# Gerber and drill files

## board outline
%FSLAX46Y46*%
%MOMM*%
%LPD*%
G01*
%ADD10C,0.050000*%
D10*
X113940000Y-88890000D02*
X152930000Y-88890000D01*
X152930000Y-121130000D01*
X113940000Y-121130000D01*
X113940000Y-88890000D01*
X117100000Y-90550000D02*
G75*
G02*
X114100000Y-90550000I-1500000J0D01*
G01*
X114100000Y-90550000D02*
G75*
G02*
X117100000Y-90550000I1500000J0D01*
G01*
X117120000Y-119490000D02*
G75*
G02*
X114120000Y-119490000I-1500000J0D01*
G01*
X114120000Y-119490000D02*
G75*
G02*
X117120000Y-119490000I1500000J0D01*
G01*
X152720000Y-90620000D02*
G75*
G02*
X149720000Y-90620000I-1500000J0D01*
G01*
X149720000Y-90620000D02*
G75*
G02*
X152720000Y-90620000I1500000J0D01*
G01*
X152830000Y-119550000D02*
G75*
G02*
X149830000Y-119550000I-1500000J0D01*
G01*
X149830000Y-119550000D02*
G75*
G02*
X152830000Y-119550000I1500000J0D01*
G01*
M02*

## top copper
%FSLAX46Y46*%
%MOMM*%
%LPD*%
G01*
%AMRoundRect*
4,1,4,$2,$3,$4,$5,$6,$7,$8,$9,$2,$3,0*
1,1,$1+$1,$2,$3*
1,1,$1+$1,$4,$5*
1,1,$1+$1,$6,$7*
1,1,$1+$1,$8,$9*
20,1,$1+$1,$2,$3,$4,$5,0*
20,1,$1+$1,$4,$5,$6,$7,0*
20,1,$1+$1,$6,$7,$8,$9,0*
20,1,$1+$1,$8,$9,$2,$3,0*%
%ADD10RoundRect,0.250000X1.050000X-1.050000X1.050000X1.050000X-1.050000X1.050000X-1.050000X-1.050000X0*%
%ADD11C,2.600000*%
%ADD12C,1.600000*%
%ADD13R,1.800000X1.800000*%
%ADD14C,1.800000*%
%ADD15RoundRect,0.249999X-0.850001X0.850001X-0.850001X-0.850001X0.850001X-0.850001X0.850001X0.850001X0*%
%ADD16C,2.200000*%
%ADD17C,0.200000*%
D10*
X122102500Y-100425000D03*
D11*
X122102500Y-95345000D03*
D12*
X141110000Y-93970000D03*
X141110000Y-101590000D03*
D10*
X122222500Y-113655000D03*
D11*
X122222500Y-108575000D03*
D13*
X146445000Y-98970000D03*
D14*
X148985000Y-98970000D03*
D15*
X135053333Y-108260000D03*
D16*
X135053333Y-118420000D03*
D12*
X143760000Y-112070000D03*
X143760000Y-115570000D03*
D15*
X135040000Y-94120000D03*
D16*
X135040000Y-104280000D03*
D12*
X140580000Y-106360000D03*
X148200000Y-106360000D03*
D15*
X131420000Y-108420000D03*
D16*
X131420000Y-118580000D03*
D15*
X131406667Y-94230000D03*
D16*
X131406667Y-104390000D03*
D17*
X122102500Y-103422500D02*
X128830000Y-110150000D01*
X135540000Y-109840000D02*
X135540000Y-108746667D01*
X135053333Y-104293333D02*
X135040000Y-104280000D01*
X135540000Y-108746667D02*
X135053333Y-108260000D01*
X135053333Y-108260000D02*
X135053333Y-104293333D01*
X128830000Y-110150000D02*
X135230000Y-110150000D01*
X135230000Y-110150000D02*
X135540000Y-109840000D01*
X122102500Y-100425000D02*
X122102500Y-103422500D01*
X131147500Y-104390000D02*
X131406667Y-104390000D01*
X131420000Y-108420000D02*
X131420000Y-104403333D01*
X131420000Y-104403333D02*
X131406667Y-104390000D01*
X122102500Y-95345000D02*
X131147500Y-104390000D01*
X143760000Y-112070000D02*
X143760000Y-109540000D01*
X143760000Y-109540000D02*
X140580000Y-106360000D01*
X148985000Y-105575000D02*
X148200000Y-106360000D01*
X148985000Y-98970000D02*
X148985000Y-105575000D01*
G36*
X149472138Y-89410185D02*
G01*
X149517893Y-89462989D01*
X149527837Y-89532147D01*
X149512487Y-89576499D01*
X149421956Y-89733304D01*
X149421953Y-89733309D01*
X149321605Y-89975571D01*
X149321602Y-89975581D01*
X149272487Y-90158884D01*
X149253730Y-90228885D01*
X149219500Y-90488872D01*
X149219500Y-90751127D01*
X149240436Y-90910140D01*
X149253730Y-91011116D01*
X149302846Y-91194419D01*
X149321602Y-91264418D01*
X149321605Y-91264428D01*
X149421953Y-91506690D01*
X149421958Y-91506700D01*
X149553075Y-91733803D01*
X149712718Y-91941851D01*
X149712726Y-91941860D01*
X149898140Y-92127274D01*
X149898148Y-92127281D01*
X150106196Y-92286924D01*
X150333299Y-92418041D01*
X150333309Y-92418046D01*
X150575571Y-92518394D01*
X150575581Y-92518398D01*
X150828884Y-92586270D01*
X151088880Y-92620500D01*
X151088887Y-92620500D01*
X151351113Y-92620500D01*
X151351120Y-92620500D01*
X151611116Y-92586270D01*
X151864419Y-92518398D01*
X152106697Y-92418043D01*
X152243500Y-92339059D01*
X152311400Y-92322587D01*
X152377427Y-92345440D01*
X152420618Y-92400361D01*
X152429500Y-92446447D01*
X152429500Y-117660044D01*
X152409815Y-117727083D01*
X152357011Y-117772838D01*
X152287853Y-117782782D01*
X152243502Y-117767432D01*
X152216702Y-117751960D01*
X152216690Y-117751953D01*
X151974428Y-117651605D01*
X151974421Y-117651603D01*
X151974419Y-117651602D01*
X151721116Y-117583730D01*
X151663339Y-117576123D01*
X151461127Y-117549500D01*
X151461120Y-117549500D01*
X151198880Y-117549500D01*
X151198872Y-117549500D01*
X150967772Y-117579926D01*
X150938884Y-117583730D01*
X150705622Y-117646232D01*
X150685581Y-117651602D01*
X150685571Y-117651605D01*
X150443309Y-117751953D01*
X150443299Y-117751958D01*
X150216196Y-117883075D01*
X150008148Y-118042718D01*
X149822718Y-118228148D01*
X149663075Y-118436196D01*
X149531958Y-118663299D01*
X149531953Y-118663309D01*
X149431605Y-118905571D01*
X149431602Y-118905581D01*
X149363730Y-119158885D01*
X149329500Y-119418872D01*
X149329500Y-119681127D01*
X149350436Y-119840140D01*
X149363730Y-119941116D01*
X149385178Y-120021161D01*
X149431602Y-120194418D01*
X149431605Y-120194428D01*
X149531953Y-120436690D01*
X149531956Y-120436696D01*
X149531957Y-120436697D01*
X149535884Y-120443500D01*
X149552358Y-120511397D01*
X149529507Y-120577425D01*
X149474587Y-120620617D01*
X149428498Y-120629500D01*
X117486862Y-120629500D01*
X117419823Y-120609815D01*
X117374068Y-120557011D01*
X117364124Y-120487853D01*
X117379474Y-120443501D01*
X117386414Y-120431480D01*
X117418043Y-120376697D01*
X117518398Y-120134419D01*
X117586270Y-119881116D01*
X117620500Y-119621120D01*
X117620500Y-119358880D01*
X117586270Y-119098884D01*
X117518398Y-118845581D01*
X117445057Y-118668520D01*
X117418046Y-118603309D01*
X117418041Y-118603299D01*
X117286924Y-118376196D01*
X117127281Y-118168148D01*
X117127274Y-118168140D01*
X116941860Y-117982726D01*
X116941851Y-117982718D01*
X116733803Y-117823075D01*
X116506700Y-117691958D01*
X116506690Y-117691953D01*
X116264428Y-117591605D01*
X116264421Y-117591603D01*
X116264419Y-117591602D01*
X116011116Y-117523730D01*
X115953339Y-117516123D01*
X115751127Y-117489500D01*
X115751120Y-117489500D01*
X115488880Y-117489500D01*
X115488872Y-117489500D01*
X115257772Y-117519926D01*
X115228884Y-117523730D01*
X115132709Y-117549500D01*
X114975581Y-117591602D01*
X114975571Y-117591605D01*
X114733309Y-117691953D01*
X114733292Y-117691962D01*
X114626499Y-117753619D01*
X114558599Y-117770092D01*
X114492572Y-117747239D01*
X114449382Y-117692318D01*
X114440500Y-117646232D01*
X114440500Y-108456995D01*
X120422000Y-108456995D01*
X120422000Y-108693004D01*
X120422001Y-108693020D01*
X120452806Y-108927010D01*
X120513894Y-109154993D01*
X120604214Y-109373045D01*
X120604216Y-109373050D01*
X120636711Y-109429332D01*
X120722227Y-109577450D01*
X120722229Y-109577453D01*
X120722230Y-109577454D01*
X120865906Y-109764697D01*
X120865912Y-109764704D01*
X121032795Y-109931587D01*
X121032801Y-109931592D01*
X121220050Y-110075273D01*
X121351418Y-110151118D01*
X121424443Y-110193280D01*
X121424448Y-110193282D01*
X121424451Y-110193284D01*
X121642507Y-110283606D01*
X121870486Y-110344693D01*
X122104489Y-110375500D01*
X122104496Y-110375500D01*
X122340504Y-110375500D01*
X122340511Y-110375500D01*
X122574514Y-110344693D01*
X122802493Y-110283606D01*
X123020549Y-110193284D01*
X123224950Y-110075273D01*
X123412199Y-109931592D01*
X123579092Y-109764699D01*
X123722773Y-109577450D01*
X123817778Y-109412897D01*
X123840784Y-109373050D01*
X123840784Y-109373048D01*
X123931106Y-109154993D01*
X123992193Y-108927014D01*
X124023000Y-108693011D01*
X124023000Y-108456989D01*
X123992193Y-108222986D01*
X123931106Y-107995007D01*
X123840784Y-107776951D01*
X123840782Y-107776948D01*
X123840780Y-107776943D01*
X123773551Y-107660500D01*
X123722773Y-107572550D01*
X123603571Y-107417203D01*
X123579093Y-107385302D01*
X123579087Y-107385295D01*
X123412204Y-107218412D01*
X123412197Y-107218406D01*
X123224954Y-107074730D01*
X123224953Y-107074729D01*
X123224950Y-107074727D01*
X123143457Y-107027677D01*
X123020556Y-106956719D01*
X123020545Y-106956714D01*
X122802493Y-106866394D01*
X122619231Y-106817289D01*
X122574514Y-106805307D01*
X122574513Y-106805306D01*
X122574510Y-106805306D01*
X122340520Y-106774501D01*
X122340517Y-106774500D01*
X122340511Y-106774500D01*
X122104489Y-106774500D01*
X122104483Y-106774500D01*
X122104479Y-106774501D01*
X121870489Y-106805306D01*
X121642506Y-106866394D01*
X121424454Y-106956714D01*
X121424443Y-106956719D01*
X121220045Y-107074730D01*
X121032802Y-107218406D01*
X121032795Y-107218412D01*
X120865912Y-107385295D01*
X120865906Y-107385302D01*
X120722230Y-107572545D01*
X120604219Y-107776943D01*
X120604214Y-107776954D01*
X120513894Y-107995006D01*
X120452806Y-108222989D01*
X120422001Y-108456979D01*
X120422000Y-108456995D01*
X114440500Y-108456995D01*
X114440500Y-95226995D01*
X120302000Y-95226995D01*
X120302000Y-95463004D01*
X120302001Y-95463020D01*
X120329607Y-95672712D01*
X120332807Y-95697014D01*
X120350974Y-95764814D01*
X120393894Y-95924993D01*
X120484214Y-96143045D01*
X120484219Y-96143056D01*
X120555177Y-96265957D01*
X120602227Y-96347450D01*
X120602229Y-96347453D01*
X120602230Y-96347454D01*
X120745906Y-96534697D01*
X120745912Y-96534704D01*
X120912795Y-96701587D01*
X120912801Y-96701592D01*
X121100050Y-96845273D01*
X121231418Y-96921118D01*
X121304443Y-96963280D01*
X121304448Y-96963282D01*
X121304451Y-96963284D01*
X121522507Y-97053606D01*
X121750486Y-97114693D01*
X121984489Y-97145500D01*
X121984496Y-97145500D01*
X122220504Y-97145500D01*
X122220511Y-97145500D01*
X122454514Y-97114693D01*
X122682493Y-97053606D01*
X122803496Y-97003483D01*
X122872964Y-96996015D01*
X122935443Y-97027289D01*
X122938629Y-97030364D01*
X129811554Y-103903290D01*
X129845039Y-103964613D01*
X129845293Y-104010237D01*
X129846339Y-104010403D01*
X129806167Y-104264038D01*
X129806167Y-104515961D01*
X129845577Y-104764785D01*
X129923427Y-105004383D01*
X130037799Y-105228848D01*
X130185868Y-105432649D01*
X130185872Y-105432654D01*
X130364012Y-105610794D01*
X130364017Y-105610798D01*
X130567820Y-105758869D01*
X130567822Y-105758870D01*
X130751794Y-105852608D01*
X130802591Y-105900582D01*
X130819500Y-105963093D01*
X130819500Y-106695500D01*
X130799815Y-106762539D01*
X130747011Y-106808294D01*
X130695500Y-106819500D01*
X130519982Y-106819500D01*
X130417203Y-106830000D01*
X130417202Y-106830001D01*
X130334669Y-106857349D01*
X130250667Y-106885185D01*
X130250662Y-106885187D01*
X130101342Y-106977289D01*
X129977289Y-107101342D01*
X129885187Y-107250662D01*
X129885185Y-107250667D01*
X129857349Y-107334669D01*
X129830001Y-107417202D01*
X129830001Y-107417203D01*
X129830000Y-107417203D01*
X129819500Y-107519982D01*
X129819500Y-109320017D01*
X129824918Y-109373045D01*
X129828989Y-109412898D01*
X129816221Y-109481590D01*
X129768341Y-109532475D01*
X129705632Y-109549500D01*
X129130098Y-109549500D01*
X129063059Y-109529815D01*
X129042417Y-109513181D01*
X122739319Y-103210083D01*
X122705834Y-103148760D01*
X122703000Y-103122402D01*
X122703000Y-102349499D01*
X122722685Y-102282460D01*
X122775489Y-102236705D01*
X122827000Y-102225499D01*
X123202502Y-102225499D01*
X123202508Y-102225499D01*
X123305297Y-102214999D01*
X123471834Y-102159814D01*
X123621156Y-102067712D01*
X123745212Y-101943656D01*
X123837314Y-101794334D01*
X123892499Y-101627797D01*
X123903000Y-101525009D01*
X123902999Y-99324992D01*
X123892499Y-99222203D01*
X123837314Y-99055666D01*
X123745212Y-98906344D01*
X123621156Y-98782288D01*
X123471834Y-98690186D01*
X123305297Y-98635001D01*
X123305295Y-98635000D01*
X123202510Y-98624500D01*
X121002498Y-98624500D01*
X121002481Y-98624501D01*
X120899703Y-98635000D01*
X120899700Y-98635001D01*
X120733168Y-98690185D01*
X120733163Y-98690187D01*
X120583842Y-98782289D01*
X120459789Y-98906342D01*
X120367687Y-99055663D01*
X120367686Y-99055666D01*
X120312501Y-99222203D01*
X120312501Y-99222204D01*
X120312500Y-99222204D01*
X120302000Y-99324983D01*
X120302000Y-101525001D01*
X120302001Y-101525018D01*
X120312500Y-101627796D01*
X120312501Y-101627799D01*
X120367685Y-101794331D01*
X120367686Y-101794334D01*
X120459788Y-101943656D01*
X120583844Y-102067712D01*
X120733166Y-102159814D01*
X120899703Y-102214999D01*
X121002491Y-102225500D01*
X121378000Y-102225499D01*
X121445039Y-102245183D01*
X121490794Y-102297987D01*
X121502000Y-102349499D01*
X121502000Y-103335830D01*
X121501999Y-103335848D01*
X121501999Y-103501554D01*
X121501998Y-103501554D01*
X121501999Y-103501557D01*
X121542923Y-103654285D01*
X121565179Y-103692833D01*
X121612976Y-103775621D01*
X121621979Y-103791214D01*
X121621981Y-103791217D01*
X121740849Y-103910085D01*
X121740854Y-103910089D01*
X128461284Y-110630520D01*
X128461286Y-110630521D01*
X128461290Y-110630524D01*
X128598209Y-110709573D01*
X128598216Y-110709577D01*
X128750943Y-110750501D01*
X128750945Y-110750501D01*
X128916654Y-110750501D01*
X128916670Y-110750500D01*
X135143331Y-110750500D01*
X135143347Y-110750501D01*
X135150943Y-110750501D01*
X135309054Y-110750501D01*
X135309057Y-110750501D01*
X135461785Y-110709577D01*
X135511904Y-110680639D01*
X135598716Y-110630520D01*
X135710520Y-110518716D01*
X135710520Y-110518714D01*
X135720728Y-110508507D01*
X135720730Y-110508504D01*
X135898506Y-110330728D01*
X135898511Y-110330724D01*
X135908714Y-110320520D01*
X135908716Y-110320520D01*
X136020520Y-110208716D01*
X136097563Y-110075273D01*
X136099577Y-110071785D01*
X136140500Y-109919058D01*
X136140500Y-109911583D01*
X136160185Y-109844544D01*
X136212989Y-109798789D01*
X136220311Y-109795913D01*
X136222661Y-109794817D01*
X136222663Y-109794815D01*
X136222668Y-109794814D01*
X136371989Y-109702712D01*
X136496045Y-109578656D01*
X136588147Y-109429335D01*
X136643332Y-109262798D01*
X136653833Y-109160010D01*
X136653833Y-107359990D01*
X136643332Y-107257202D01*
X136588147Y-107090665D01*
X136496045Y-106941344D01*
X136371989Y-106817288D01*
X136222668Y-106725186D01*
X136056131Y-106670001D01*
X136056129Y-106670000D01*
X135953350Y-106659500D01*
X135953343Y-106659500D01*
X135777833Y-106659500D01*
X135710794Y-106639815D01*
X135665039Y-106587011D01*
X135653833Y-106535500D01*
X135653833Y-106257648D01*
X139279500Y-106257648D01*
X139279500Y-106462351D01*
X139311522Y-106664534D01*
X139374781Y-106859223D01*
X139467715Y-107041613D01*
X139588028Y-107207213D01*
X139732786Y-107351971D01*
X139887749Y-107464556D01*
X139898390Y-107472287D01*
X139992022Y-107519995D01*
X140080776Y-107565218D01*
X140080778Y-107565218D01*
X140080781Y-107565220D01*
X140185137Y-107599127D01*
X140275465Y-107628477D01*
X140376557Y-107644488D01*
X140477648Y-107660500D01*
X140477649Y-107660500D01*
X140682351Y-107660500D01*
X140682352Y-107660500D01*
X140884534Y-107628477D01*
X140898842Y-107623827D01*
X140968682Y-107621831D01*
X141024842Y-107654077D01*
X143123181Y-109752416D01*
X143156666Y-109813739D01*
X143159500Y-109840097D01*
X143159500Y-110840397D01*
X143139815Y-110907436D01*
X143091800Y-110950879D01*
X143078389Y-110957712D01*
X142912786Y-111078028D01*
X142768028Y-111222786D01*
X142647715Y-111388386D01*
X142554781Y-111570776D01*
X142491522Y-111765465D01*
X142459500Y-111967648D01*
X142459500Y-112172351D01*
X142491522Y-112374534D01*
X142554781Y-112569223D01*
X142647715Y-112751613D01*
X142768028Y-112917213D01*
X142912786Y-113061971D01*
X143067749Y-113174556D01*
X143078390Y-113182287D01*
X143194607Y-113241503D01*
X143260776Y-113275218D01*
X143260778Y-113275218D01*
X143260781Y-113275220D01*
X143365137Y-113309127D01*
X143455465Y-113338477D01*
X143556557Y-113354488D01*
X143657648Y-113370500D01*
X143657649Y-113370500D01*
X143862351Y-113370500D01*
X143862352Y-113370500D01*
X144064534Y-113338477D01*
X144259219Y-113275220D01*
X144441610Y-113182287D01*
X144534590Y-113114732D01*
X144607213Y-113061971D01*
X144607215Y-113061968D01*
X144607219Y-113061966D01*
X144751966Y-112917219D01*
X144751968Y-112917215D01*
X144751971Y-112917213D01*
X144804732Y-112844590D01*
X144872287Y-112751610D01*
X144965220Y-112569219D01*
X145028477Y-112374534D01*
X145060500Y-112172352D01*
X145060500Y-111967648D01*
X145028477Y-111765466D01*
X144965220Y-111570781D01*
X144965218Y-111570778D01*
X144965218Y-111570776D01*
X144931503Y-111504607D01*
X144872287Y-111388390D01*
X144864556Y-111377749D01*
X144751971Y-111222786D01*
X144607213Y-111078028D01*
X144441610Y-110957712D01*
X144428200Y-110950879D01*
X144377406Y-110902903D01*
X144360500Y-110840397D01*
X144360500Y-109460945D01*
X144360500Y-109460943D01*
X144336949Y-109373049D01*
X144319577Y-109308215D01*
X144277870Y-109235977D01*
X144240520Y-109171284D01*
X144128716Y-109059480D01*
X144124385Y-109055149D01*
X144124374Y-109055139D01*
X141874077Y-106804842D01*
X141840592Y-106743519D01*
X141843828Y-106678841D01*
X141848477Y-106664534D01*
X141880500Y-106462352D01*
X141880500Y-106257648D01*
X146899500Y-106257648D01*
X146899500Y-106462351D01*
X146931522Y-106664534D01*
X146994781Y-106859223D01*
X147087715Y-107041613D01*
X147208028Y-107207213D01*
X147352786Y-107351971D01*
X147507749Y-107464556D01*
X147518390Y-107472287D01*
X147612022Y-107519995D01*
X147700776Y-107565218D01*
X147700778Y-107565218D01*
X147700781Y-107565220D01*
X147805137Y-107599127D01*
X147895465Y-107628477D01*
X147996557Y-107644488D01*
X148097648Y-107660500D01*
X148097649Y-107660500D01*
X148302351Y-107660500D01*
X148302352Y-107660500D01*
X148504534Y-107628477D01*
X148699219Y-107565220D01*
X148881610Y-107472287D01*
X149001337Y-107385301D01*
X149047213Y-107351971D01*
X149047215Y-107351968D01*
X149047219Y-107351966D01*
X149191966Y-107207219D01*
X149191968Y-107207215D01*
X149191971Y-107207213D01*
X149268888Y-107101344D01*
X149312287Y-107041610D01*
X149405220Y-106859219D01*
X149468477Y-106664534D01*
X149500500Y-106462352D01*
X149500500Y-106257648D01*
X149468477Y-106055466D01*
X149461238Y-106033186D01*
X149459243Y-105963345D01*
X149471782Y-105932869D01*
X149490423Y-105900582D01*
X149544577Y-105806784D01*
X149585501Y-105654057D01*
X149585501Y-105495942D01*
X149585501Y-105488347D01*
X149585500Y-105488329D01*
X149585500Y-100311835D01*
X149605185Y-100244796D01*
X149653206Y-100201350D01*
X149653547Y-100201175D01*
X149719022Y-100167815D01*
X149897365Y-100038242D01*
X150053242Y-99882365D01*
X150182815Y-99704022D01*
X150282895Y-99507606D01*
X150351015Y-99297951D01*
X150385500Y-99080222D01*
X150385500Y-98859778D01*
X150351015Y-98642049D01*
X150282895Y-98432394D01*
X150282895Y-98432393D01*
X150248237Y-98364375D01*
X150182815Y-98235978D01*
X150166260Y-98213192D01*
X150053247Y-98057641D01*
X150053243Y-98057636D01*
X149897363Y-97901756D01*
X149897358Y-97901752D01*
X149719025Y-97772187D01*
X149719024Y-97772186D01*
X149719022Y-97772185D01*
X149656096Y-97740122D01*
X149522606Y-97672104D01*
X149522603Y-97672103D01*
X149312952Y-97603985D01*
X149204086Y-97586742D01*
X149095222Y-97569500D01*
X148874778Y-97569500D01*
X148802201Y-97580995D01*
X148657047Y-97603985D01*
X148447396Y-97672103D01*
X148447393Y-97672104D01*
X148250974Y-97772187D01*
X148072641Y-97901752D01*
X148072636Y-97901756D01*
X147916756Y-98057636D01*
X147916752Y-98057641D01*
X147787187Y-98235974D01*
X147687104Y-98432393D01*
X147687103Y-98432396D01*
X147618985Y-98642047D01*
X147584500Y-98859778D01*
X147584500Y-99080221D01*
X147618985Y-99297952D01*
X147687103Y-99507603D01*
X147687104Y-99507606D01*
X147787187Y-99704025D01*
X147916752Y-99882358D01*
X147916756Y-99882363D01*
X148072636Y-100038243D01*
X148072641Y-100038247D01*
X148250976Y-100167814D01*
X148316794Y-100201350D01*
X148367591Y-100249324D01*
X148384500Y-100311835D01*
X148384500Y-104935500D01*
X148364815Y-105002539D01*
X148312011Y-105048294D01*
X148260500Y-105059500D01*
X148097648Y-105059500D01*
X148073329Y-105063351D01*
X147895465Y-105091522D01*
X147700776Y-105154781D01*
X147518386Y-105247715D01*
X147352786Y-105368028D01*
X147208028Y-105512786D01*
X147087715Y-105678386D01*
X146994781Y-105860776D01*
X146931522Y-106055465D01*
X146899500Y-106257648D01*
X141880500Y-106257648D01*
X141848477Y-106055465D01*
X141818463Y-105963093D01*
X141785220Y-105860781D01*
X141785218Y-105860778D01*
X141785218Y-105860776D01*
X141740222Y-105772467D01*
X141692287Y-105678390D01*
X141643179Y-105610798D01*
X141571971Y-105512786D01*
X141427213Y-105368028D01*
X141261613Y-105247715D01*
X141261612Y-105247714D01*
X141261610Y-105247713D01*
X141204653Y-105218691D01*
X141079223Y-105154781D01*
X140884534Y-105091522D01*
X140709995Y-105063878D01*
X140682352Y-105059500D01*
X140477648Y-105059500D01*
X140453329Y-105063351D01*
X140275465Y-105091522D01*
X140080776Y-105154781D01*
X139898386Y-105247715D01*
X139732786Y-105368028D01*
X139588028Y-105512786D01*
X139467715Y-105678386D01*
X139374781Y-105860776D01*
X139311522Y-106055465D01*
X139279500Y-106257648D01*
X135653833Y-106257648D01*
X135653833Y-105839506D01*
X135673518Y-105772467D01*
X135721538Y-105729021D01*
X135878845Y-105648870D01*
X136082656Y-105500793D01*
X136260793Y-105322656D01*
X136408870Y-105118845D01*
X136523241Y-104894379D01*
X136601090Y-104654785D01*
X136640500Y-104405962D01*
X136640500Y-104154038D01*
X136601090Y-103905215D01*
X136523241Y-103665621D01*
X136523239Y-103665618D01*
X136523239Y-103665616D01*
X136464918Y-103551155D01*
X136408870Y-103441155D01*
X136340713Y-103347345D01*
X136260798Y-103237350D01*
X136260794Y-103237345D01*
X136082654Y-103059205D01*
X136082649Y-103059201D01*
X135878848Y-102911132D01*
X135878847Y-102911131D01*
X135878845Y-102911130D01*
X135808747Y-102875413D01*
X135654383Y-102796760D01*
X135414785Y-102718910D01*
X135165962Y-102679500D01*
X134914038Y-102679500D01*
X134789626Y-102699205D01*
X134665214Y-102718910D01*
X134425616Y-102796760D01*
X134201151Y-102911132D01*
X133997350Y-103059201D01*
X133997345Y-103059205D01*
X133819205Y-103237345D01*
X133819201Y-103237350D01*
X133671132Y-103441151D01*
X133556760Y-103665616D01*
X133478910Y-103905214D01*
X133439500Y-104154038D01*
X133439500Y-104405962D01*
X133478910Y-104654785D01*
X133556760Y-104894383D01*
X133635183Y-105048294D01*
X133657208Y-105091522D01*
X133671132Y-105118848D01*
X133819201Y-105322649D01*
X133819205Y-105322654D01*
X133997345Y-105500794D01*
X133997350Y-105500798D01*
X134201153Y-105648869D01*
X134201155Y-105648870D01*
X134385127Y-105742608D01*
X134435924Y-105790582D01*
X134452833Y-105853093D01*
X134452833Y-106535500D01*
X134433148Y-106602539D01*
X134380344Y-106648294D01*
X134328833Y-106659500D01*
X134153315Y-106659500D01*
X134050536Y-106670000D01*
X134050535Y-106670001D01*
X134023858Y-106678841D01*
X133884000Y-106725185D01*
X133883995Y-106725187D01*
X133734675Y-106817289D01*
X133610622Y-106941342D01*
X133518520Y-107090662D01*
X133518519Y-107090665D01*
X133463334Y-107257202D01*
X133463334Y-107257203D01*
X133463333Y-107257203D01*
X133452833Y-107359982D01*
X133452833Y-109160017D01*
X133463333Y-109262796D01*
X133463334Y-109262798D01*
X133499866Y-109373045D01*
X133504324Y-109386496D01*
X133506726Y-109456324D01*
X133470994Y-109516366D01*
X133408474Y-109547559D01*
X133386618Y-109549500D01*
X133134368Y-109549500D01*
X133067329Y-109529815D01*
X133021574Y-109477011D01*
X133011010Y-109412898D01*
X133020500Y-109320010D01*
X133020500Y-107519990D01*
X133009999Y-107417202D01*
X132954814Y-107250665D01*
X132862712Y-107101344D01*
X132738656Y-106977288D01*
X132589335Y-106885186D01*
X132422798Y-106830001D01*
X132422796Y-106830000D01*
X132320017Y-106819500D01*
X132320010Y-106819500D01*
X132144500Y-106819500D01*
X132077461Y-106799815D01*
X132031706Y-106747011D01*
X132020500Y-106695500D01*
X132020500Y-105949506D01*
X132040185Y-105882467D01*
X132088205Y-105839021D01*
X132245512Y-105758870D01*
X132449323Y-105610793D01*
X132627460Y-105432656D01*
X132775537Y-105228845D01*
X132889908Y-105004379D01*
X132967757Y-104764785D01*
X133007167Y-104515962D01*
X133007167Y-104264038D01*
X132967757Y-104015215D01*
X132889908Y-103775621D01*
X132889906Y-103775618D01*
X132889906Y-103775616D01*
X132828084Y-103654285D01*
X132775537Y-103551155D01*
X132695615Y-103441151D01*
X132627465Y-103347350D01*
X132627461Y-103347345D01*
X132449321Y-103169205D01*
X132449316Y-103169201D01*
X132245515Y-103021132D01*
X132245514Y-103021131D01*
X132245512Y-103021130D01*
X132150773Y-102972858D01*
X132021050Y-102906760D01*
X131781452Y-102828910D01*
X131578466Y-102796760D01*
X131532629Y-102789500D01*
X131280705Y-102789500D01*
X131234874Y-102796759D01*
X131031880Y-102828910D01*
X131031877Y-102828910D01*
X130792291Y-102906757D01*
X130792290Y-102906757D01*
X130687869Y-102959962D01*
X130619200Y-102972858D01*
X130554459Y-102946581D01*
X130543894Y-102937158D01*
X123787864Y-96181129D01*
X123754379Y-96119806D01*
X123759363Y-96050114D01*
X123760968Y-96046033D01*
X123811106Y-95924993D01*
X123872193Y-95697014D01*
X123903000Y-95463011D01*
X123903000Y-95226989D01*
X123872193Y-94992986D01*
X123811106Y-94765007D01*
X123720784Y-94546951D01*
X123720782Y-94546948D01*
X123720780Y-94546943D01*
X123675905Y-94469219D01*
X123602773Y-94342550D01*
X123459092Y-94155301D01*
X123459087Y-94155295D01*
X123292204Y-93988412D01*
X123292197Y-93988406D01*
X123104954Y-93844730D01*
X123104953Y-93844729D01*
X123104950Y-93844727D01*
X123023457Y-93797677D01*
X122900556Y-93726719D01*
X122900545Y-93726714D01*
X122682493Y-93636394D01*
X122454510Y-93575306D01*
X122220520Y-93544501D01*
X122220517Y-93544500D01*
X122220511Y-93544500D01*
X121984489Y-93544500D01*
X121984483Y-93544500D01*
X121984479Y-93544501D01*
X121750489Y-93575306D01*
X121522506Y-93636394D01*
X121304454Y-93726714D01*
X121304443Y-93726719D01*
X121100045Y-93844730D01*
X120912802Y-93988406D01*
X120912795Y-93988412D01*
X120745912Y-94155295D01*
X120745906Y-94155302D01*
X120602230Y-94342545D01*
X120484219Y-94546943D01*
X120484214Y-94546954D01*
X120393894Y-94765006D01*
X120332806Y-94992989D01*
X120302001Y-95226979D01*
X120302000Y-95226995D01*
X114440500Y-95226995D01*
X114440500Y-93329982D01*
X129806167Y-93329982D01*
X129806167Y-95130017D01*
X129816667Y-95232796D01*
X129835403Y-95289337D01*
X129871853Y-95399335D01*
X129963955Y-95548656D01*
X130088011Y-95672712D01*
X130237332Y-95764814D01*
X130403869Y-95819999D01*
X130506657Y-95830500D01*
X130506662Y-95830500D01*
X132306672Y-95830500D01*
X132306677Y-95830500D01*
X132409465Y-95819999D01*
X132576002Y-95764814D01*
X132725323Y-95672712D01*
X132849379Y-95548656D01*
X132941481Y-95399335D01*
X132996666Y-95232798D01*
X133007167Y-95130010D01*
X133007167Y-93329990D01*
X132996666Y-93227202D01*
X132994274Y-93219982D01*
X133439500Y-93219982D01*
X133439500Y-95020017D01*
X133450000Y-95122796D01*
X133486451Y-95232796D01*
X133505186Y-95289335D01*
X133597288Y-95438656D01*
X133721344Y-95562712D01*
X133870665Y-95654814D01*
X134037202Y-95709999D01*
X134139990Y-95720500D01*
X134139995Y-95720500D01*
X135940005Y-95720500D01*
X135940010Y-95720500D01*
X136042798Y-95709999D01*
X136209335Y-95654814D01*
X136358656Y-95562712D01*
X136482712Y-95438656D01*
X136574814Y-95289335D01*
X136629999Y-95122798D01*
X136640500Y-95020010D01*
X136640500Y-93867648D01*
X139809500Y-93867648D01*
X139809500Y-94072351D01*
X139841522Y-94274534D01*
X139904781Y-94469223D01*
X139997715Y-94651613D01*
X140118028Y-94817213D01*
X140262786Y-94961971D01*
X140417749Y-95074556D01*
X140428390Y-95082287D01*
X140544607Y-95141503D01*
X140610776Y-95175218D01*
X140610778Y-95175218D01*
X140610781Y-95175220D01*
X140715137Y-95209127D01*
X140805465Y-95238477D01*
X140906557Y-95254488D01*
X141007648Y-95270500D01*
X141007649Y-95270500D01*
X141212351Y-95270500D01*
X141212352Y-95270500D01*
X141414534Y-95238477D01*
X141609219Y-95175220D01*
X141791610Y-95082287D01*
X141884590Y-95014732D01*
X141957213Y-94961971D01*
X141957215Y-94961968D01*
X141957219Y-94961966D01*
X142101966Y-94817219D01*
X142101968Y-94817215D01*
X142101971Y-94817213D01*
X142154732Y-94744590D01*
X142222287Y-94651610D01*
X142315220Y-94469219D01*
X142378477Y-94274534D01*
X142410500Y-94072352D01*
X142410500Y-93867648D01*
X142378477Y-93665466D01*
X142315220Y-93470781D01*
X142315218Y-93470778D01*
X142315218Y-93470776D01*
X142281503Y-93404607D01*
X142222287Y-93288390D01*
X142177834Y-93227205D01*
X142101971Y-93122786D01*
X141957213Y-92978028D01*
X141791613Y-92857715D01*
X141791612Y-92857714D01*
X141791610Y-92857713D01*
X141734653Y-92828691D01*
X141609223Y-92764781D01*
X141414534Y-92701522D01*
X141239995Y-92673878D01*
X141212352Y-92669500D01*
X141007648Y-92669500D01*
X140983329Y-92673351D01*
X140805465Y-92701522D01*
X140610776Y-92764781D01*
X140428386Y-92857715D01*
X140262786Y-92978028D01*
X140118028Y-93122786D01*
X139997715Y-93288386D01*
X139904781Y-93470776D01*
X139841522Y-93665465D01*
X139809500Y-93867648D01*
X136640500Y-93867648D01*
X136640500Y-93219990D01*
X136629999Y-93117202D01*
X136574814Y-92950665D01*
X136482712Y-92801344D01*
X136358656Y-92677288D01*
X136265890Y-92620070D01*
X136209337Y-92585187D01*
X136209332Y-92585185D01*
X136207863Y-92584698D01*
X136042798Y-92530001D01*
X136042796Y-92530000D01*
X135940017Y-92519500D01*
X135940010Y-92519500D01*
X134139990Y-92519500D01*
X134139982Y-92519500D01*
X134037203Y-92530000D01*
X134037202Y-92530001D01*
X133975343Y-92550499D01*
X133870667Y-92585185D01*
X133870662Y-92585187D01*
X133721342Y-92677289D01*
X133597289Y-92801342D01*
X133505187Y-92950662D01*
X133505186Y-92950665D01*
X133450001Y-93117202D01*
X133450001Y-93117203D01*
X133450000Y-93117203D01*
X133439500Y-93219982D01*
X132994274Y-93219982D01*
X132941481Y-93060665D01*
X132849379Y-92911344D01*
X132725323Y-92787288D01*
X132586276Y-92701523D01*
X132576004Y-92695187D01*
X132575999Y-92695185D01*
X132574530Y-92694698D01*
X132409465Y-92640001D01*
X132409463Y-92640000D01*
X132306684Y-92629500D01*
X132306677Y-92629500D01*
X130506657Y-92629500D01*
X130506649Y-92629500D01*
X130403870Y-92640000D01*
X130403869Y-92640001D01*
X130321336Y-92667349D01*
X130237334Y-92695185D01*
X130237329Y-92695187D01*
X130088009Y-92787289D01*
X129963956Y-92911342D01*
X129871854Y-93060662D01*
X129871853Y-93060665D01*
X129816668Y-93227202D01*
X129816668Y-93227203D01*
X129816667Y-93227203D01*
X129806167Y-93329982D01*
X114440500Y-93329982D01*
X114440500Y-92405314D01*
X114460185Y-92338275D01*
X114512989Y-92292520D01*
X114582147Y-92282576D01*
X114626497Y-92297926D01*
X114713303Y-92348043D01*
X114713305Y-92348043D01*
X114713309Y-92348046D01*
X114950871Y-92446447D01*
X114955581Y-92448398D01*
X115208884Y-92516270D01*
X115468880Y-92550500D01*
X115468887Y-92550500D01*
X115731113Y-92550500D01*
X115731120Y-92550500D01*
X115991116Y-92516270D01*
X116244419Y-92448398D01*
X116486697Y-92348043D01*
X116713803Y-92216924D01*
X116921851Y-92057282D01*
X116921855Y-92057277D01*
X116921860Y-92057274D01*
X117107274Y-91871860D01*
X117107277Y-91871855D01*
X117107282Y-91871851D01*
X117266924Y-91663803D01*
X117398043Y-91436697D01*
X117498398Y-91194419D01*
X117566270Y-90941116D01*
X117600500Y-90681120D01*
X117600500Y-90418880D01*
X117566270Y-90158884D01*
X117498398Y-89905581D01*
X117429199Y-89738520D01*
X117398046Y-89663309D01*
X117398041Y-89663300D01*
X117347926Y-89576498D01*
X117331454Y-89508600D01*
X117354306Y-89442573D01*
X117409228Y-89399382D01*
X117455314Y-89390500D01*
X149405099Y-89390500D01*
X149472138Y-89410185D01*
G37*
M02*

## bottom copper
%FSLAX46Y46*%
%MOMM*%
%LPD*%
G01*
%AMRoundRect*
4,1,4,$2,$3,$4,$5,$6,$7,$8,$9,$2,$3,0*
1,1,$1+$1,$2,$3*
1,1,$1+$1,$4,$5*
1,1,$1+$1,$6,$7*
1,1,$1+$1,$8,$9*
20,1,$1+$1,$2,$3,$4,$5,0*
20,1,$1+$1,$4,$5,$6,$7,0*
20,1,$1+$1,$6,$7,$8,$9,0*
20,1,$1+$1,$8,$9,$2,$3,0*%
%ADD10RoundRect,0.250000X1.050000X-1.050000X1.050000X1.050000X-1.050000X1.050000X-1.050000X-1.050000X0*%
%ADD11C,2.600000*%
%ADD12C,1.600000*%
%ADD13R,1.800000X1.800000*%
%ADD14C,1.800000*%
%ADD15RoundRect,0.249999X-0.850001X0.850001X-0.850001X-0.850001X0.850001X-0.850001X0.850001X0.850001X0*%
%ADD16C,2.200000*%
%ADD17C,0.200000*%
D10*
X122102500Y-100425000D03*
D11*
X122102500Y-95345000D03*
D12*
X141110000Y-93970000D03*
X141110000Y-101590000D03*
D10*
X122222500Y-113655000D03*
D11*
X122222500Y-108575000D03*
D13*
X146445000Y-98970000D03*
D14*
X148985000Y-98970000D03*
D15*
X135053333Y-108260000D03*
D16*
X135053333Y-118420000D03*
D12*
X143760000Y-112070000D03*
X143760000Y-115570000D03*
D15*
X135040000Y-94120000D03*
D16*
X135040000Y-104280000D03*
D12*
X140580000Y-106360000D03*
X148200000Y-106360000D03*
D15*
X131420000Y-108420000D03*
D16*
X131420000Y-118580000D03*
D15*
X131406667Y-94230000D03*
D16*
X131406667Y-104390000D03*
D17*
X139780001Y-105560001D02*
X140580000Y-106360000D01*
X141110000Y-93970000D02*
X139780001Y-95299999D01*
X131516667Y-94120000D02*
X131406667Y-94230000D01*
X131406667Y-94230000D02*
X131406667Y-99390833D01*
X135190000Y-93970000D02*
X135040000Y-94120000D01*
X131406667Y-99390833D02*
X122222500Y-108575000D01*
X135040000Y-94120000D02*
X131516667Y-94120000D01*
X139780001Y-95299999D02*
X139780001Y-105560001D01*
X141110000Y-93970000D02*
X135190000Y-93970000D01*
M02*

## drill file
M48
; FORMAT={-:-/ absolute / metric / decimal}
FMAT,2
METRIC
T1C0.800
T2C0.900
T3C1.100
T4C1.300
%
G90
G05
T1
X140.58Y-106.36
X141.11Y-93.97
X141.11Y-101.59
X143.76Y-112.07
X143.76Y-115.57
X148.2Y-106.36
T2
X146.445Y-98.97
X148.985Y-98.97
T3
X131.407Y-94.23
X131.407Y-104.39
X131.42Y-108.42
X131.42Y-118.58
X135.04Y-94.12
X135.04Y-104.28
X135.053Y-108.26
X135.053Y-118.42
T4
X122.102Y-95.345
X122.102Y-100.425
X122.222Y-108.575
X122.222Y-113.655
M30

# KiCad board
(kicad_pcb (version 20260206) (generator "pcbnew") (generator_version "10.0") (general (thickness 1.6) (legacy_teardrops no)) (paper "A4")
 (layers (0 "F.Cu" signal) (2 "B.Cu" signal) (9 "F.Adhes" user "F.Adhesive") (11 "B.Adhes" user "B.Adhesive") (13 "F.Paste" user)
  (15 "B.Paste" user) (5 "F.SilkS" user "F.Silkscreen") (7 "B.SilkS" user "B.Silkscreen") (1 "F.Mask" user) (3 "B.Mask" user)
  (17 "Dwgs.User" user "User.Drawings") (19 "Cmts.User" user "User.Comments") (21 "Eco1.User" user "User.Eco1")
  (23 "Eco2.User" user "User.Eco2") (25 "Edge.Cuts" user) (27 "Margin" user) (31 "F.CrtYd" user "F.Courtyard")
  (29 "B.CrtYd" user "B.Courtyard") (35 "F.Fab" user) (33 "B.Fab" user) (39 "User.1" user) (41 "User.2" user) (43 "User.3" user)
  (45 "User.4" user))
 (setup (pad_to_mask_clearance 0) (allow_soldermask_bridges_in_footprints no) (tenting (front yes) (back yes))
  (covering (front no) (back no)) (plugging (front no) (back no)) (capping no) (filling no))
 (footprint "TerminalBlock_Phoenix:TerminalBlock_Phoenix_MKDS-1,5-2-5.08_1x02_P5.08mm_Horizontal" (layer "F.Cu") (at 122.1025 100.425 90)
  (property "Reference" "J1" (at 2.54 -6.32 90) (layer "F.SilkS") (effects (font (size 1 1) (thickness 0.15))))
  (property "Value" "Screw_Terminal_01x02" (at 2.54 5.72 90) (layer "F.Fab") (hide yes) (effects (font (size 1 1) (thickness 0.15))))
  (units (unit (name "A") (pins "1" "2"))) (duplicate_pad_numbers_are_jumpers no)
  (pad "1" thru_hole roundrect (at 0 0 90) (size 2.6 2.6) (drill 1.3) (layers "*.Cu" "*.Mask") (remove_unused_layers no)
   (roundrect_rratio 0.096154) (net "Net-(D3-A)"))
  (pad "2" thru_hole circle (at 5.08 0 90) (size 2.6 2.6) (drill 1.3) (layers "*.Cu" "*.Mask") (remove_unused_layers no) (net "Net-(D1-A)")))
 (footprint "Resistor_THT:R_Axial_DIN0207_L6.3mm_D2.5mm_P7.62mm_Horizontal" (layer "F.Cu") (at 141.11 93.97 -90)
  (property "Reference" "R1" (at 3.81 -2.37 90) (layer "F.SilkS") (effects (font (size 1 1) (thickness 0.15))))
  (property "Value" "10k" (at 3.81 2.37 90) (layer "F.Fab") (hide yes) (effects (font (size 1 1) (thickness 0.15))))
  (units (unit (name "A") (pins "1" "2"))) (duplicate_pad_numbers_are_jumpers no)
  (pad "1" thru_hole circle (at 0 0 270) (size 1.6 1.6) (drill 0.8) (layers "*.Cu" "*.Mask") (remove_unused_layers no) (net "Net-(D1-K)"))
  (pad "2" thru_hole circle (at 7.62 0 270) (size 1.6 1.6) (drill 0.8) (layers "*.Cu" "*.Mask") (remove_unused_layers no) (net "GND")))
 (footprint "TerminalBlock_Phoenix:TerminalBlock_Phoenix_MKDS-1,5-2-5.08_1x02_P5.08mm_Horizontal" (layer "F.Cu") (at 122.2225 113.655 90)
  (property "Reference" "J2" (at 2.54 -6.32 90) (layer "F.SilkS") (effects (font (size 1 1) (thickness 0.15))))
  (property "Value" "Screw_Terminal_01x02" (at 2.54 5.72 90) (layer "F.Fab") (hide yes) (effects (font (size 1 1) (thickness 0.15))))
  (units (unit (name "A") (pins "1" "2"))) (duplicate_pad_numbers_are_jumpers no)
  (pad "1" thru_hole roundrect (at 0 0 90) (size 2.6 2.6) (drill 1.3) (layers "*.Cu" "*.Mask") (remove_unused_layers no)
   (roundrect_rratio 0.096154) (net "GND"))
  (pad "2" thru_hole circle (at 5.08 0 90) (size 2.6 2.6) (drill 1.3) (layers "*.Cu" "*.Mask") (remove_unused_layers no) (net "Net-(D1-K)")))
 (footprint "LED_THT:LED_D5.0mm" (layer "F.Cu") (at 146.445 98.97)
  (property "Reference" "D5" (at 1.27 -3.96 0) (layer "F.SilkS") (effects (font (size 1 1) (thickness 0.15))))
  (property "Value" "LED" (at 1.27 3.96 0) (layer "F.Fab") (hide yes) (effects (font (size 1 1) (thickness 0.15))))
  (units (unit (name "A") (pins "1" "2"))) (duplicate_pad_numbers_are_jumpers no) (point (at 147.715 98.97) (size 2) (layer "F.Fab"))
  (pad "1" thru_hole rect (at 0 0) (size 1.8 1.8) (drill 0.9) (layers "*.Cu" "*.Mask") (remove_unused_layers no) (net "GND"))
  (pad "2" thru_hole circle (at 2.54 0) (size 1.8 1.8) (drill 0.9) (layers "*.Cu" "*.Mask") (remove_unused_layers no) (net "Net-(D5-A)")))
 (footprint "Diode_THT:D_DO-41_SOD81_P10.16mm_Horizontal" (layer "F.Cu") (at 135.053333 108.26 -90)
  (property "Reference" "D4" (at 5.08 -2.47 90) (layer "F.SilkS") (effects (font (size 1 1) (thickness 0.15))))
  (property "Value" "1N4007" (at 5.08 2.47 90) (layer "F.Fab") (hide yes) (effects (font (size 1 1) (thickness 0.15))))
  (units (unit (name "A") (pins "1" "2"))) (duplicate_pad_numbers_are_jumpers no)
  (pad "1" thru_hole roundrect (at 0 0 270) (size 2.2 2.2) (drill 1.1) (layers "*.Cu" "*.Mask") (remove_unused_layers no)
   (roundrect_rratio 0.113636) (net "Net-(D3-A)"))
  (pad "2" thru_hole circle (at 10.16 0 270) (size 2.2 2.2) (drill 1.1) (layers "*.Cu" "*.Mask") (remove_unused_layers no) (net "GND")))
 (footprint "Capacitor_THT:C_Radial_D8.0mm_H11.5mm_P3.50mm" (layer "F.Cu") (at 143.76 112.07 -90)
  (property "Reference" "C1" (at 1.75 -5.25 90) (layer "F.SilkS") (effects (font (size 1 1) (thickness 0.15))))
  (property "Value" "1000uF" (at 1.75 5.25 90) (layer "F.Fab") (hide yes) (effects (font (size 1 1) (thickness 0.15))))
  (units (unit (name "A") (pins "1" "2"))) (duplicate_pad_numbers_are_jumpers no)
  (pad "1" thru_hole circle (at 0 0 270) (size 1.6 1.6) (drill 0.8) (layers "*.Cu" "*.Mask") (remove_unused_layers no) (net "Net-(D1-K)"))
  (pad "2" thru_hole circle (at 3.5 0 270) (size 1.6 1.6) (drill 0.8) (layers "*.Cu" "*.Mask") (remove_unused_layers no) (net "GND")))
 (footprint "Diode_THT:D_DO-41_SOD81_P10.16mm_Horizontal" (layer "F.Cu") (at 135.04 94.12 -90)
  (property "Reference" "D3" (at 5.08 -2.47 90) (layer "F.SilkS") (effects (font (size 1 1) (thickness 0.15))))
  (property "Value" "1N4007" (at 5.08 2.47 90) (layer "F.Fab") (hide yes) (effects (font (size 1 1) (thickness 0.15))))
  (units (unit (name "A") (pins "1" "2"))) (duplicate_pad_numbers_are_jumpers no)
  (pad "1" thru_hole roundrect (at 0 0 270) (size 2.2 2.2) (drill 1.1) (layers "*.Cu" "*.Mask") (remove_unused_layers no)
   (roundrect_rratio 0.113636) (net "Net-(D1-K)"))
  (pad "2" thru_hole circle (at 10.16 0 270) (size 2.2 2.2) (drill 1.1) (layers "*.Cu" "*.Mask") (remove_unused_layers no)
   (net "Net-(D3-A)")))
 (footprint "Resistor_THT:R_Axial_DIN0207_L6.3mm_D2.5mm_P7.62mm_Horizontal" (layer "F.Cu") (at 140.58 106.36)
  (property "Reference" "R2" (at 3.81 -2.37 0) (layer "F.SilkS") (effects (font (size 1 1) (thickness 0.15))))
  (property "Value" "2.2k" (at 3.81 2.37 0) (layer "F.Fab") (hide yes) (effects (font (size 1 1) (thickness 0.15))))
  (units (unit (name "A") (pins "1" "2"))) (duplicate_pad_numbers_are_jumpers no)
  (pad "1" thru_hole circle (at 0 0) (size 1.6 1.6) (drill 0.8) (layers "*.Cu" "*.Mask") (remove_unused_layers no) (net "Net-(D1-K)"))
  (pad "2" thru_hole circle (at 7.62 0) (size 1.6 1.6) (drill 0.8) (layers "*.Cu" "*.Mask") (remove_unused_layers no) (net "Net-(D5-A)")))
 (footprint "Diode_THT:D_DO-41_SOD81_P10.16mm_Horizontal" (layer "F.Cu") (at 131.42 108.42 -90)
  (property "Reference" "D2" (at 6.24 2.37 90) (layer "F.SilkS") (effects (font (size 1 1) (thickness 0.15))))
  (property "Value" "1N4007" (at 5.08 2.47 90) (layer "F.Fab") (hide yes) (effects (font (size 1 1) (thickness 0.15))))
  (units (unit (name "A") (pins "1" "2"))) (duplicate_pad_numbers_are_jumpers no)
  (pad "1" thru_hole roundrect (at 0 0 270) (size 2.2 2.2) (drill 1.1) (layers "*.Cu" "*.Mask") (remove_unused_layers no)
   (roundrect_rratio 0.113636) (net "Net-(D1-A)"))
  (pad "2" thru_hole circle (at 10.16 0 270) (size 2.2 2.2) (drill 1.1) (layers "*.Cu" "*.Mask") (remove_unused_layers no) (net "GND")))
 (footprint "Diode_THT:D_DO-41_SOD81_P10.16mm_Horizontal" (layer "F.Cu") (at 131.406667 94.23 -90)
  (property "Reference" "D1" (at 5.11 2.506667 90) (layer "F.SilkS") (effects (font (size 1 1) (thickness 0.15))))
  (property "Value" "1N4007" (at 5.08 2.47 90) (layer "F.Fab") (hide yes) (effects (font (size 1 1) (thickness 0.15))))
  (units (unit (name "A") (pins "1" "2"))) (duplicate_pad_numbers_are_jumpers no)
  (pad "1" thru_hole roundrect (at 0 0 270) (size 2.2 2.2) (drill 1.1) (layers "*.Cu" "*.Mask") (remove_unused_layers no)
   (roundrect_rratio 0.113636) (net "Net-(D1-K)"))
  (pad "2" thru_hole circle (at 10.16 0 270) (size 2.2 2.2) (drill 1.1) (layers "*.Cu" "*.Mask") (remove_unused_layers no)
   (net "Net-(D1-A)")))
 (gr_rect (start 113.94 88.89) (end 152.93 121.13) (stroke (width 0.05) (type default)) (fill no) (layer "Edge.Cuts"))
 (gr_circle (center 115.6 90.55) (end 117.1 90.55) (stroke (width 0.05) (type default)) (fill no) (layer "Edge.Cuts"))
 (gr_circle (center 115.62 119.49) (end 117.12 119.49) (stroke (width 0.05) (type default)) (fill no) (layer "Edge.Cuts"))
 (gr_circle (center 151.22 90.62) (end 152.72 90.62) (stroke (width 0.05) (type default)) (fill no) (layer "Edge.Cuts"))
 (gr_circle (center 151.33 119.55) (end 152.83 119.55) (stroke (width 0.05) (type default)) (fill no) (layer "Edge.Cuts"))
 (segment (start 122.1025 103.4225) (end 128.83 110.15) (width 0.2) (layer "F.Cu") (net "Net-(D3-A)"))
 (segment (start 135.54 109.84) (end 135.54 108.746667) (width 0.2) (layer "F.Cu") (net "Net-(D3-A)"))
 (segment (start 135.053333 104.293333) (end 135.04 104.28) (width 0.2) (layer "F.Cu") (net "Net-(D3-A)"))
 (segment (start 135.54 108.746667) (end 135.053333 108.26) (width 0.2) (layer "F.Cu") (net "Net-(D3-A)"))
 (segment (start 135.053333 108.26) (end 135.053333 104.293333) (width 0.2) (layer "F.Cu") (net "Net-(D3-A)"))
 (segment (start 128.83 110.15) (end 135.23 110.15) (width 0.2) (layer "F.Cu") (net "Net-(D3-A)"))
 (segment (start 135.23 110.15) (end 135.54 109.84) (width 0.2) (layer "F.Cu") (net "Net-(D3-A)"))
 (segment (start 122.1025 100.425) (end 122.1025 103.4225) (width 0.2) (layer "F.Cu") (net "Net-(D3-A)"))
 (segment (start 131.1475 104.39) (end 131.406667 104.39) (width 0.2) (layer "F.Cu") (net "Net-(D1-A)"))
 (segment (start 131.42 108.42) (end 131.42 104.403333) (width 0.2) (layer "F.Cu") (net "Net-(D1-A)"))
 (segment (start 131.42 104.403333) (end 131.406667 104.39) (width 0.2) (layer "F.Cu") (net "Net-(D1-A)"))
 (segment (start 122.1025 95.345) (end 131.1475 104.39) (width 0.2) (layer "F.Cu") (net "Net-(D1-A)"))
 (segment (start 143.76 112.07) (end 143.76 109.54) (width 0.2) (layer "F.Cu") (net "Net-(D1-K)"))
 (segment (start 143.76 109.54) (end 140.58 106.36) (width 0.2) (layer "F.Cu") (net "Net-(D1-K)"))
 (segment (start 139.780001 105.560001) (end 140.58 106.36) (width 0.2) (layer "B.Cu") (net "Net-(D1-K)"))
 (segment (start 141.11 93.97) (end 139.780001 95.299999) (width 0.2) (layer "B.Cu") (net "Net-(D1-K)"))
 (segment (start 131.516667 94.12) (end 131.406667 94.23) (width 0.2) (layer "B.Cu") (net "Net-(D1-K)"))
 (segment (start 131.406667 94.23) (end 131.406667 99.390833) (width 0.2) (layer "B.Cu") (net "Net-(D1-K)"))
 (segment (start 135.19 93.97) (end 135.04 94.12) (width 0.2) (layer "B.Cu") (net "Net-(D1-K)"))
 (segment (start 131.406667 99.390833) (end 122.2225 108.575) (width 0.2) (layer "B.Cu") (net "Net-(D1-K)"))
 (segment (start 135.04 94.12) (end 131.516667 94.12) (width 0.2) (layer "B.Cu") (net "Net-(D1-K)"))
 (segment (start 139.780001 95.299999) (end 139.780001 105.560001) (width 0.2) (layer "B.Cu") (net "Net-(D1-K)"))
 (segment (start 141.11 93.97) (end 135.19 93.97) (width 0.2) (layer "B.Cu") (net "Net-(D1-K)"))
 (segment (start 148.985 105.575) (end 148.2 106.36) (width 0.2) (layer "F.Cu") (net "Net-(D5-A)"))
 (segment (start 148.985 98.97) (end 148.985 105.575) (width 0.2) (layer "F.Cu") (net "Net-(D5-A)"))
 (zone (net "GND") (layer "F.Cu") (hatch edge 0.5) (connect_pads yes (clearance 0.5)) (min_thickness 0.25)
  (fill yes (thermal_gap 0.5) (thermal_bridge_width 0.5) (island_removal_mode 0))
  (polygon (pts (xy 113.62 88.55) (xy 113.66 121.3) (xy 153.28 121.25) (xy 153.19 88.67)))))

